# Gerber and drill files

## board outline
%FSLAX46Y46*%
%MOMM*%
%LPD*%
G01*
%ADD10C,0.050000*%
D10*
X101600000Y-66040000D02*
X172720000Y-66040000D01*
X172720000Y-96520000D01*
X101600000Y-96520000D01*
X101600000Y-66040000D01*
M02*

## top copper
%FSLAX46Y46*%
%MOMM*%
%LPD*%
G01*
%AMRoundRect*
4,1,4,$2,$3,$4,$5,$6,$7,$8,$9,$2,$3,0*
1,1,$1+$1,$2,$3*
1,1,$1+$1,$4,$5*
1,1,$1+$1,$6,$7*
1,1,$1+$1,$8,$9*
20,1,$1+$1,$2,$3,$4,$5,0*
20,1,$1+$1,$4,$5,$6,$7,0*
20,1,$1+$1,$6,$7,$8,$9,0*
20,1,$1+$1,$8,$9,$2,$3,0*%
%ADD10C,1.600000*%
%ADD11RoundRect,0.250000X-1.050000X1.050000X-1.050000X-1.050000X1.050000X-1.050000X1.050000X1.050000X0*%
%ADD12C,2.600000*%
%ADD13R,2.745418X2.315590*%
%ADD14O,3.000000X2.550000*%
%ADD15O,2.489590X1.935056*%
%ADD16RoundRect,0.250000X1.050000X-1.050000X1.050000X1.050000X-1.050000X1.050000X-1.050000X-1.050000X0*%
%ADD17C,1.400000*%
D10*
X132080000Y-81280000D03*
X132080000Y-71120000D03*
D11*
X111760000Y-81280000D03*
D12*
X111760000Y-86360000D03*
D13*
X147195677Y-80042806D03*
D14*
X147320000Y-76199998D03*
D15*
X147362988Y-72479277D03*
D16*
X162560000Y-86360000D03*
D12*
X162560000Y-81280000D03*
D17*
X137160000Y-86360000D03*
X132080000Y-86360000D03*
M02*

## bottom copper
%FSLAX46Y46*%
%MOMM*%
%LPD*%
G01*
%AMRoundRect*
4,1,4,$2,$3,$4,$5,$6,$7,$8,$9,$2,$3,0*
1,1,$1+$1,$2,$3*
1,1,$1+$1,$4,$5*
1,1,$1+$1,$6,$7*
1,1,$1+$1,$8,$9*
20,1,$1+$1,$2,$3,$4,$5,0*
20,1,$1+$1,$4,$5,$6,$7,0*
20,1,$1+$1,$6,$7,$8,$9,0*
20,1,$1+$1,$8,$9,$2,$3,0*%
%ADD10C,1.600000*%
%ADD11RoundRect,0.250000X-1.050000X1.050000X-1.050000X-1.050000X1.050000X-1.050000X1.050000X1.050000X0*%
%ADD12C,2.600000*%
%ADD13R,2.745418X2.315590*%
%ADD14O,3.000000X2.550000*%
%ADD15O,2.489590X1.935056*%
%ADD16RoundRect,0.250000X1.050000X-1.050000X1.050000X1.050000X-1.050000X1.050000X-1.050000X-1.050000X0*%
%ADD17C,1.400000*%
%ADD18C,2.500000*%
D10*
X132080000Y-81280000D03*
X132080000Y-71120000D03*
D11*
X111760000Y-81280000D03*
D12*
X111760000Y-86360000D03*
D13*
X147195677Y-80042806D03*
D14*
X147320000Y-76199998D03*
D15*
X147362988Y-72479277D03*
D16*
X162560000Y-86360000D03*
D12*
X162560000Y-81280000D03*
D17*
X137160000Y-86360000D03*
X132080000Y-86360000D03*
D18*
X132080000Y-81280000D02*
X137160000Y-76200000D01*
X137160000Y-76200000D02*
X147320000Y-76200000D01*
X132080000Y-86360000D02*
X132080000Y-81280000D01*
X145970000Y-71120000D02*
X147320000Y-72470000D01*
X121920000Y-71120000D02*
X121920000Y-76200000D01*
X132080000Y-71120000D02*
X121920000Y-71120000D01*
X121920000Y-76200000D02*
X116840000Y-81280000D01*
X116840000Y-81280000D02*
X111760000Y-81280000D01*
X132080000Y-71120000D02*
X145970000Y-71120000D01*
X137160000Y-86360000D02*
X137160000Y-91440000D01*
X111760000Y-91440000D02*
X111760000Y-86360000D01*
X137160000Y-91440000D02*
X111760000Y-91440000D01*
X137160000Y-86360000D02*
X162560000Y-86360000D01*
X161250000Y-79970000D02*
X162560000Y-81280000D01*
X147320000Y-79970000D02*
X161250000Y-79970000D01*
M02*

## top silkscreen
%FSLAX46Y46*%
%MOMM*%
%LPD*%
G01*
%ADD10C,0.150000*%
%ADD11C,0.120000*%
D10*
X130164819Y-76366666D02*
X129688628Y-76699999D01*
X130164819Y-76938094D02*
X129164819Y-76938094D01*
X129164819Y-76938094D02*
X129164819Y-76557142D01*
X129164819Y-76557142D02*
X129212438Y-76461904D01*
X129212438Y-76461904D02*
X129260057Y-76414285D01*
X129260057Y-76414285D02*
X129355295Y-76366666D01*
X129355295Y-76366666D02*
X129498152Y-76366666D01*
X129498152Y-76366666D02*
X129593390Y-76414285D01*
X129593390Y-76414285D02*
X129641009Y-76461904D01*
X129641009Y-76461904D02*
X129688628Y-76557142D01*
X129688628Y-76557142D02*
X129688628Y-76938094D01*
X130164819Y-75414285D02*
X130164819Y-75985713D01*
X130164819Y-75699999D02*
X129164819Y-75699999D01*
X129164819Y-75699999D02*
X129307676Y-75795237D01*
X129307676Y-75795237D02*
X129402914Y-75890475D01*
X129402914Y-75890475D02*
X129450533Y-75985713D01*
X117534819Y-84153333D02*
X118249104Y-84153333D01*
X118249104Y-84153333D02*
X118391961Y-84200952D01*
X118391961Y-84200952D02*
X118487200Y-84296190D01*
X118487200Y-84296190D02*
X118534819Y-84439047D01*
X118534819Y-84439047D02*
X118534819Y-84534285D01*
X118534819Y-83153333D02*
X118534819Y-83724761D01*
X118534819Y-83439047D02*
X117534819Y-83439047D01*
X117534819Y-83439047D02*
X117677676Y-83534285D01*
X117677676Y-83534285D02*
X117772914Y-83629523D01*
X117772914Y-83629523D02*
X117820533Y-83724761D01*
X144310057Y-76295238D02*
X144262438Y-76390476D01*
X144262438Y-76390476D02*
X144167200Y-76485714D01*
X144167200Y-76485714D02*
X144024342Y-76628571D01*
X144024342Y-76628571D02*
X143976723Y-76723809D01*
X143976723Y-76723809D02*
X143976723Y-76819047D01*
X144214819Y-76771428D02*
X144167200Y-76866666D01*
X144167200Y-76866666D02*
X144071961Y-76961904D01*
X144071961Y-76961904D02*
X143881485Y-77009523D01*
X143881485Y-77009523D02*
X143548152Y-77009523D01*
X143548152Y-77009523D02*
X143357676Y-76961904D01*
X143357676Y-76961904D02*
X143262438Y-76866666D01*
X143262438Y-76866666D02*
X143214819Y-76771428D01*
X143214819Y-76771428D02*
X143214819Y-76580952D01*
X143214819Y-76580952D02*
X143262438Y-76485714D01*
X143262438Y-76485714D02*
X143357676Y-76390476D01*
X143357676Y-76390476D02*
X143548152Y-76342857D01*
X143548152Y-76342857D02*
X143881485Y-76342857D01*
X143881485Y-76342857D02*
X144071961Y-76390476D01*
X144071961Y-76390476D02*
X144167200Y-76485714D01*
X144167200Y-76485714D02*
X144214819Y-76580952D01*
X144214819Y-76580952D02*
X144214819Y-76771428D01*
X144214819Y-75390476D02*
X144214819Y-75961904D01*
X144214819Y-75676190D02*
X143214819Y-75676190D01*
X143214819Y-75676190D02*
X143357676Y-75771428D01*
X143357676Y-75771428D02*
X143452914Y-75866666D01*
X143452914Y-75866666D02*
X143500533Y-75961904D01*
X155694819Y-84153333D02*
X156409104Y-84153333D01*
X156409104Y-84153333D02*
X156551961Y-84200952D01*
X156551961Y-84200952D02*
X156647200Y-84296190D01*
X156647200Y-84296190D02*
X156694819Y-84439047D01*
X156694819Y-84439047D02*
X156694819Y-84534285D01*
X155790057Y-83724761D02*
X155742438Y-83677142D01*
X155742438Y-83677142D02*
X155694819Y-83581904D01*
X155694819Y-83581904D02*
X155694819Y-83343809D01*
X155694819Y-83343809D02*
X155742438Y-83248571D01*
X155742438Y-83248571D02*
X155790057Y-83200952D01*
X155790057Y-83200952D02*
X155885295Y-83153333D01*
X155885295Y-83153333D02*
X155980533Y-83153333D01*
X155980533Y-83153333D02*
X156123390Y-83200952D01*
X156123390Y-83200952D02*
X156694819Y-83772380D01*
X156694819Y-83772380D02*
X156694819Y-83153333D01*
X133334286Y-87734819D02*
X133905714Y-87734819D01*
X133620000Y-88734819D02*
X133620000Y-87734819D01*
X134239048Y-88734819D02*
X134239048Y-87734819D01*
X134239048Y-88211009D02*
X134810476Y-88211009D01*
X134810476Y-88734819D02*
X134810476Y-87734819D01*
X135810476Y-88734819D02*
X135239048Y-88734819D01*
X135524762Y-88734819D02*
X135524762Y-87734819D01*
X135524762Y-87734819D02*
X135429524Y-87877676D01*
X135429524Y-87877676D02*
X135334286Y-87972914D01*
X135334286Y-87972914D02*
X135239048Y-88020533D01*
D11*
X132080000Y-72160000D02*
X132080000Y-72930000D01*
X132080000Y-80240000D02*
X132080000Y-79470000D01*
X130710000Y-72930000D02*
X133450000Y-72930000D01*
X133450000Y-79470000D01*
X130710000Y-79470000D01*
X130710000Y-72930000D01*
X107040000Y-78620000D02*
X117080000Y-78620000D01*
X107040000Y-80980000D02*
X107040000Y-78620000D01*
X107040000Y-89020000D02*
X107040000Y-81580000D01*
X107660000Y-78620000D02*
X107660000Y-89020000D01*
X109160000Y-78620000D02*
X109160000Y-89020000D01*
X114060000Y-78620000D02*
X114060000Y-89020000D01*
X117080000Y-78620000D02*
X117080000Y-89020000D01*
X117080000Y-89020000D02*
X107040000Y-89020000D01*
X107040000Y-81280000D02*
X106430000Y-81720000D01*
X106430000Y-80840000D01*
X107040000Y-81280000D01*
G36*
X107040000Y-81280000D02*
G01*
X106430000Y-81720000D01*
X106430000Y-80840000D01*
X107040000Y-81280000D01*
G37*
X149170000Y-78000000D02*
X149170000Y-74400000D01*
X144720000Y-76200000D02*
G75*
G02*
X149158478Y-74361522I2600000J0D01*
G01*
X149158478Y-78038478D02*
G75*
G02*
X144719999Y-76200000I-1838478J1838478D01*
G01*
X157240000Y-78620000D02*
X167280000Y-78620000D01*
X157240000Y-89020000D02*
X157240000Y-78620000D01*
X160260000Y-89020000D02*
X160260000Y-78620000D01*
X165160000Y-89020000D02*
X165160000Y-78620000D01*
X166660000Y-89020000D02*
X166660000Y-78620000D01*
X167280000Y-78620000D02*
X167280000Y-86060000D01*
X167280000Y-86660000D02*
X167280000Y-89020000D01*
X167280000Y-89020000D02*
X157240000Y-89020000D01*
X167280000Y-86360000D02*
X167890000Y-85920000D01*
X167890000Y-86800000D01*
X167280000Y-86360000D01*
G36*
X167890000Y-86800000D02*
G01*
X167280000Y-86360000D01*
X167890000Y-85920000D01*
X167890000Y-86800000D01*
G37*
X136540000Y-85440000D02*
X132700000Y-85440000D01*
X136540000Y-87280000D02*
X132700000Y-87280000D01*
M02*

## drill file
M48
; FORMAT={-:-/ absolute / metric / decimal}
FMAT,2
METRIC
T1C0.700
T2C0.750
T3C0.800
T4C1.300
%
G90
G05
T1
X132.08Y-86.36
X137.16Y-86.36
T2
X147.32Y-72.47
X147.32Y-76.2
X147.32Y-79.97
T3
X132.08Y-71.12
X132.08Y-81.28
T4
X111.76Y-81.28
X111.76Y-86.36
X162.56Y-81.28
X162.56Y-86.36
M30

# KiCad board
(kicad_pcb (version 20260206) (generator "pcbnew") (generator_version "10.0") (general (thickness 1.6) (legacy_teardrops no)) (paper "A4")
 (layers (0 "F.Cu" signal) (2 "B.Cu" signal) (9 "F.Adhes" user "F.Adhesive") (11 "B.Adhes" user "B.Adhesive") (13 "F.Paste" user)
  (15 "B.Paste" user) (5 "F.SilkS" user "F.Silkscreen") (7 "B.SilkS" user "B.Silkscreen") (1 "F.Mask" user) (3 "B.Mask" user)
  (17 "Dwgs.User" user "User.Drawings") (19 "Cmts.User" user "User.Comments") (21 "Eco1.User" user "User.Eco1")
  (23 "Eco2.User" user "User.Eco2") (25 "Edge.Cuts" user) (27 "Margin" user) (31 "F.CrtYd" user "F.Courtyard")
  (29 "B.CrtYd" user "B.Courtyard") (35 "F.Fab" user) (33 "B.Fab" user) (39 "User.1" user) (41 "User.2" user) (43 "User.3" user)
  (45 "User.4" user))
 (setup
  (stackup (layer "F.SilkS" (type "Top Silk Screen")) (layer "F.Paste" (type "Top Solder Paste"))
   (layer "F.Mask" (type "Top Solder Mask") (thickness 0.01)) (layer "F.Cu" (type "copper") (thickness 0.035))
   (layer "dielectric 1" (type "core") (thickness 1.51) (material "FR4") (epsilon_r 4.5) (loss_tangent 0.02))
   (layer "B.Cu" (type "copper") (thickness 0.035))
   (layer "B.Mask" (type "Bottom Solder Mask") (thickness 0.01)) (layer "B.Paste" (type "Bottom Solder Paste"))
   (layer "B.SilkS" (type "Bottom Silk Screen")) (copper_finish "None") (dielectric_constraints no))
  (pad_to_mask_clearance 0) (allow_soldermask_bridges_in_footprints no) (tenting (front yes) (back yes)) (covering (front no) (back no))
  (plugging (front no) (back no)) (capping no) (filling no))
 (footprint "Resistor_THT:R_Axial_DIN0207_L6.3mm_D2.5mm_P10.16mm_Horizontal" (layer "F.Cu") (at 132.08 81.28 90)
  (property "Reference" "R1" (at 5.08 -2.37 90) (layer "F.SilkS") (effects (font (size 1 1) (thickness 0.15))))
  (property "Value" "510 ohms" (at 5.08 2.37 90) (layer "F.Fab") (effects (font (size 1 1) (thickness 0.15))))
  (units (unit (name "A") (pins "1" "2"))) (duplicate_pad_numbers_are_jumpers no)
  (fp_line (start 9.12 0) (end 8.35 0) (stroke (width 0.12) (type solid)) (layer "F.SilkS"))
  (fp_line (start 1.04 0) (end 1.81 0) (stroke (width 0.12) (type solid)) (layer "F.SilkS"))
  (fp_rect (start 1.81 -1.37) (end 8.35 1.37) (stroke (width 0.12) (type solid)) (fill no) (layer "F.SilkS"))
  (pad "1" thru_hole circle (at 0 0 90) (size 1.6 1.6) (drill 0.8) (layers "*.Cu" "*.Mask") (remove_unused_layers no) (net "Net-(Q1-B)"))
  (pad "2" thru_hole circle (at 10.16 0 90) (size 1.6 1.6) (drill 0.8) (layers "*.Cu" "*.Mask") (remove_unused_layers no)
   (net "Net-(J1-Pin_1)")))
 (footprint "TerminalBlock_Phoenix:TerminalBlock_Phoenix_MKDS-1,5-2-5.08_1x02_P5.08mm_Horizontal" (layer "F.Cu") (at 111.76 81.28 -90)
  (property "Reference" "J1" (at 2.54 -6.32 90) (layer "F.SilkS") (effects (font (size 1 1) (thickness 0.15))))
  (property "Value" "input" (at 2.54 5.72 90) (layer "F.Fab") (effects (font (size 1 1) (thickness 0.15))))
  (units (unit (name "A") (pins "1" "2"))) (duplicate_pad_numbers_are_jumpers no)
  (fp_line (start -2.66 4.72) (end -2.66 -5.32) (stroke (width 0.12) (type solid)) (layer "F.SilkS"))
  (fp_line (start -0.3 4.72) (end -2.66 4.72) (stroke (width 0.12) (type solid)) (layer "F.SilkS"))
  (fp_line (start 7.74 4.72) (end 0.3 4.72) (stroke (width 0.12) (type solid)) (layer "F.SilkS"))
  (fp_line (start -2.66 4.1) (end 7.74 4.1) (stroke (width 0.12) (type solid)) (layer "F.SilkS"))
  (fp_line (start -2.66 2.6) (end 7.74 2.6) (stroke (width 0.12) (type solid)) (layer "F.SilkS"))
  (fp_line (start -2.66 -2.3) (end 7.74 -2.3) (stroke (width 0.12) (type solid)) (layer "F.SilkS"))
  (fp_line (start -2.66 -5.32) (end 7.74 -5.32) (stroke (width 0.12) (type solid)) (layer "F.SilkS"))
  (fp_line (start 7.74 -5.32) (end 7.74 4.72) (stroke (width 0.12) (type solid)) (layer "F.SilkS"))
  (fp_poly (pts (xy 0 4.72) (xy 0.44 5.33) (xy -0.44 5.33)) (stroke (width 0.12) (type solid)) (fill yes) (layer "F.SilkS"))
  (pad "1" thru_hole roundrect (at 0 0 270) (size 2.6 2.6) (drill 1.3) (layers "*.Cu" "*.Mask") (remove_unused_layers no)
   (roundrect_rratio 0.096154) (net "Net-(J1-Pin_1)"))
  (pad "2" thru_hole circle (at 5.08 0 270) (size 2.6 2.6) (drill 1.3) (layers "*.Cu" "*.Mask") (remove_unused_layers no)
   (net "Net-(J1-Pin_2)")))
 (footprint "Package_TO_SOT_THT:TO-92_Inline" (layer "F.Cu") (at 147.32 77.47 90)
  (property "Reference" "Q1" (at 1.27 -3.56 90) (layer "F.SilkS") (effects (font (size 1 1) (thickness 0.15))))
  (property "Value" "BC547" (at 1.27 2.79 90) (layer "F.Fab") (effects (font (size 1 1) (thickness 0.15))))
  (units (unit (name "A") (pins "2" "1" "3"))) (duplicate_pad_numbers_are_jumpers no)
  (fp_line (start -0.53 1.85) (end 3.07 1.85) (stroke (width 0.12) (type solid)) (layer "F.SilkS"))
  (fp_arc (start 1.27 -2.6) (mid 3.672087 -0.994977) (end 3.108478 1.838478) (stroke (width 0.12) (type solid)) (layer "F.SilkS"))
  (fp_arc (start -0.568478 1.838478) (mid -1.132087 -0.994977) (end 1.27 -2.6) (stroke (width 0.12) (type solid)) (layer "F.SilkS"))
  (pad "1" thru_hole rect (at -2.5 0 90) (size 2.31559 2.745418) (drill 0.75 (offset -0.072806 -0.124323)) (layers "*.Cu" "*.Mask")
   (remove_unused_layers no) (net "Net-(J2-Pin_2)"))
  (pad "2" thru_hole oval (at 1.27 0 90) (size 2.55 3) (drill 0.75 (offset 0.000002 0)) (layers "*.Cu" "*.Mask") (remove_unused_layers no)
   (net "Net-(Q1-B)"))
  (pad "3" thru_hole oval (at 5 0 90) (size 1.935056 2.48959) (drill 0.75 (offset -0.009277 0.042988)) (layers "*.Cu" "*.Mask")
   (remove_unused_layers no) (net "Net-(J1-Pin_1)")))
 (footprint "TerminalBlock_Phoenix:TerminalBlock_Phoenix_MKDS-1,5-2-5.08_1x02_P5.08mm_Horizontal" (layer "F.Cu") (at 162.56 86.36 90)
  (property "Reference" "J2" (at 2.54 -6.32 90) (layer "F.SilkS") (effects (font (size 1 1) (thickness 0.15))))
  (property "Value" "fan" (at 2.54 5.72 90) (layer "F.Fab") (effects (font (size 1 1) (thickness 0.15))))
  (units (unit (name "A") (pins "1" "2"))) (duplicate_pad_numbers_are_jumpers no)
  (fp_line (start 7.74 -5.32) (end 7.74 4.72) (stroke (width 0.12) (type solid)) (layer "F.SilkS"))
  (fp_line (start -2.66 -5.32) (end 7.74 -5.32) (stroke (width 0.12) (type solid)) (layer "F.SilkS"))
  (fp_line (start -2.66 -2.3) (end 7.74 -2.3) (stroke (width 0.12) (type solid)) (layer "F.SilkS"))
  (fp_line (start -2.66 2.6) (end 7.74 2.6) (stroke (width 0.12) (type solid)) (layer "F.SilkS"))
  (fp_line (start -2.66 4.1) (end 7.74 4.1) (stroke (width 0.12) (type solid)) (layer "F.SilkS"))
  (fp_line (start 7.74 4.72) (end 0.3 4.72) (stroke (width 0.12) (type solid)) (layer "F.SilkS"))
  (fp_line (start -0.3 4.72) (end -2.66 4.72) (stroke (width 0.12) (type solid)) (layer "F.SilkS"))
  (fp_line (start -2.66 4.72) (end -2.66 -5.32) (stroke (width 0.12) (type solid)) (layer "F.SilkS"))
  (fp_poly (pts (xy 0 4.72) (xy 0.44 5.33) (xy -0.44 5.33)) (stroke (width 0.12) (type solid)) (fill yes) (layer "F.SilkS"))
  (pad "1" thru_hole roundrect (at 0 0 90) (size 2.6 2.6) (drill 1.3) (layers "*.Cu" "*.Mask") (remove_unused_layers no)
   (roundrect_rratio 0.096154) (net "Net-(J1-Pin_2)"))
  (pad "2" thru_hole circle (at 5.08 0 90) (size 2.6 2.6) (drill 1.3) (layers "*.Cu" "*.Mask") (remove_unused_layers no)
   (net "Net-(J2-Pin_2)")))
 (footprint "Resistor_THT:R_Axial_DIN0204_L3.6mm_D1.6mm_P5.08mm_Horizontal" (layer "F.Cu") (at 137.16 86.36 180)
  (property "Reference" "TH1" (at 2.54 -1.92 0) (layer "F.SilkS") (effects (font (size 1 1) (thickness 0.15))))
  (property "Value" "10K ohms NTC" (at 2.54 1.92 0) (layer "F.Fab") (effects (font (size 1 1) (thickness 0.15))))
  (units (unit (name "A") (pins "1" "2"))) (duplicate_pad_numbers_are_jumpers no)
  (fp_line (start 0.62 0.92) (end 4.46 0.92) (stroke (width 0.12) (type solid)) (layer "F.SilkS"))
  (fp_line (start 0.62 -0.92) (end 4.46 -0.92) (stroke (width 0.12) (type solid)) (layer "F.SilkS"))
  (pad "1" thru_hole circle (at 0 0 180) (size 1.4 1.4) (drill 0.7) (layers "*.Cu" "*.Mask") (remove_unused_layers no)
   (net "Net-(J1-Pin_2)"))
  (pad "2" thru_hole circle (at 5.08 0 180) (size 1.4 1.4) (drill 0.7) (layers "*.Cu" "*.Mask") (remove_unused_layers no) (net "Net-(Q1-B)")))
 (gr_rect (start 101.6 66.04) (end 172.72 96.52) (stroke (width 0.05) (type default)) (fill no) (layer "Edge.Cuts"))
 (segment (start 132.08 81.28) (end 137.16 76.2) (width 2.5) (layer "B.Cu") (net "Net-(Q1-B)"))
 (segment (start 137.16 76.2) (end 147.32 76.2) (width 2.5) (layer "B.Cu") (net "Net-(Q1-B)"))
 (segment (start 132.08 86.36) (end 132.08 81.28) (width 2.5) (layer "B.Cu") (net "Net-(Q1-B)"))
 (segment (start 145.97 71.12) (end 147.32 72.47) (width 2.5) (layer "B.Cu") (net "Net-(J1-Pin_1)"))
 (segment (start 121.92 71.12) (end 121.92 76.2) (width 2.5) (layer "B.Cu") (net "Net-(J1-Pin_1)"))
 (segment (start 132.08 71.12) (end 121.92 71.12) (width 2.5) (layer "B.Cu") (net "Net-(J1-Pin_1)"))
 (segment (start 121.92 76.2) (end 116.84 81.28) (width 2.5) (layer "B.Cu") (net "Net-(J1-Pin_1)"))
 (segment (start 116.84 81.28) (end 111.76 81.28) (width 2.5) (layer "B.Cu") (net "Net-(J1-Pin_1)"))
 (segment (start 132.08 71.12) (end 145.97 71.12) (width 2.5) (layer "B.Cu") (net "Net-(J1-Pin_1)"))
 (segment (start 137.16 86.36) (end 137.16 91.44) (width 2.5) (layer "B.Cu") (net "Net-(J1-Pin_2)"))
 (segment (start 111.76 91.44) (end 111.76 86.36) (width 2.5) (layer "B.Cu") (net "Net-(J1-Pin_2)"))
 (segment (start 137.16 91.44) (end 111.76 91.44) (width 2.5) (layer "B.Cu") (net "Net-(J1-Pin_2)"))
 (segment (start 137.16 86.36) (end 162.56 86.36) (width 2.5) (layer "B.Cu") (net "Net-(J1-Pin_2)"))
 (segment (start 161.25 79.97) (end 162.56 81.28) (width 2.5) (layer "B.Cu") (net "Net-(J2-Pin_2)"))
 (segment (start 147.32 79.97) (end 161.25 79.97) (width 2.5) (layer "B.Cu") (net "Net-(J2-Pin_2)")))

